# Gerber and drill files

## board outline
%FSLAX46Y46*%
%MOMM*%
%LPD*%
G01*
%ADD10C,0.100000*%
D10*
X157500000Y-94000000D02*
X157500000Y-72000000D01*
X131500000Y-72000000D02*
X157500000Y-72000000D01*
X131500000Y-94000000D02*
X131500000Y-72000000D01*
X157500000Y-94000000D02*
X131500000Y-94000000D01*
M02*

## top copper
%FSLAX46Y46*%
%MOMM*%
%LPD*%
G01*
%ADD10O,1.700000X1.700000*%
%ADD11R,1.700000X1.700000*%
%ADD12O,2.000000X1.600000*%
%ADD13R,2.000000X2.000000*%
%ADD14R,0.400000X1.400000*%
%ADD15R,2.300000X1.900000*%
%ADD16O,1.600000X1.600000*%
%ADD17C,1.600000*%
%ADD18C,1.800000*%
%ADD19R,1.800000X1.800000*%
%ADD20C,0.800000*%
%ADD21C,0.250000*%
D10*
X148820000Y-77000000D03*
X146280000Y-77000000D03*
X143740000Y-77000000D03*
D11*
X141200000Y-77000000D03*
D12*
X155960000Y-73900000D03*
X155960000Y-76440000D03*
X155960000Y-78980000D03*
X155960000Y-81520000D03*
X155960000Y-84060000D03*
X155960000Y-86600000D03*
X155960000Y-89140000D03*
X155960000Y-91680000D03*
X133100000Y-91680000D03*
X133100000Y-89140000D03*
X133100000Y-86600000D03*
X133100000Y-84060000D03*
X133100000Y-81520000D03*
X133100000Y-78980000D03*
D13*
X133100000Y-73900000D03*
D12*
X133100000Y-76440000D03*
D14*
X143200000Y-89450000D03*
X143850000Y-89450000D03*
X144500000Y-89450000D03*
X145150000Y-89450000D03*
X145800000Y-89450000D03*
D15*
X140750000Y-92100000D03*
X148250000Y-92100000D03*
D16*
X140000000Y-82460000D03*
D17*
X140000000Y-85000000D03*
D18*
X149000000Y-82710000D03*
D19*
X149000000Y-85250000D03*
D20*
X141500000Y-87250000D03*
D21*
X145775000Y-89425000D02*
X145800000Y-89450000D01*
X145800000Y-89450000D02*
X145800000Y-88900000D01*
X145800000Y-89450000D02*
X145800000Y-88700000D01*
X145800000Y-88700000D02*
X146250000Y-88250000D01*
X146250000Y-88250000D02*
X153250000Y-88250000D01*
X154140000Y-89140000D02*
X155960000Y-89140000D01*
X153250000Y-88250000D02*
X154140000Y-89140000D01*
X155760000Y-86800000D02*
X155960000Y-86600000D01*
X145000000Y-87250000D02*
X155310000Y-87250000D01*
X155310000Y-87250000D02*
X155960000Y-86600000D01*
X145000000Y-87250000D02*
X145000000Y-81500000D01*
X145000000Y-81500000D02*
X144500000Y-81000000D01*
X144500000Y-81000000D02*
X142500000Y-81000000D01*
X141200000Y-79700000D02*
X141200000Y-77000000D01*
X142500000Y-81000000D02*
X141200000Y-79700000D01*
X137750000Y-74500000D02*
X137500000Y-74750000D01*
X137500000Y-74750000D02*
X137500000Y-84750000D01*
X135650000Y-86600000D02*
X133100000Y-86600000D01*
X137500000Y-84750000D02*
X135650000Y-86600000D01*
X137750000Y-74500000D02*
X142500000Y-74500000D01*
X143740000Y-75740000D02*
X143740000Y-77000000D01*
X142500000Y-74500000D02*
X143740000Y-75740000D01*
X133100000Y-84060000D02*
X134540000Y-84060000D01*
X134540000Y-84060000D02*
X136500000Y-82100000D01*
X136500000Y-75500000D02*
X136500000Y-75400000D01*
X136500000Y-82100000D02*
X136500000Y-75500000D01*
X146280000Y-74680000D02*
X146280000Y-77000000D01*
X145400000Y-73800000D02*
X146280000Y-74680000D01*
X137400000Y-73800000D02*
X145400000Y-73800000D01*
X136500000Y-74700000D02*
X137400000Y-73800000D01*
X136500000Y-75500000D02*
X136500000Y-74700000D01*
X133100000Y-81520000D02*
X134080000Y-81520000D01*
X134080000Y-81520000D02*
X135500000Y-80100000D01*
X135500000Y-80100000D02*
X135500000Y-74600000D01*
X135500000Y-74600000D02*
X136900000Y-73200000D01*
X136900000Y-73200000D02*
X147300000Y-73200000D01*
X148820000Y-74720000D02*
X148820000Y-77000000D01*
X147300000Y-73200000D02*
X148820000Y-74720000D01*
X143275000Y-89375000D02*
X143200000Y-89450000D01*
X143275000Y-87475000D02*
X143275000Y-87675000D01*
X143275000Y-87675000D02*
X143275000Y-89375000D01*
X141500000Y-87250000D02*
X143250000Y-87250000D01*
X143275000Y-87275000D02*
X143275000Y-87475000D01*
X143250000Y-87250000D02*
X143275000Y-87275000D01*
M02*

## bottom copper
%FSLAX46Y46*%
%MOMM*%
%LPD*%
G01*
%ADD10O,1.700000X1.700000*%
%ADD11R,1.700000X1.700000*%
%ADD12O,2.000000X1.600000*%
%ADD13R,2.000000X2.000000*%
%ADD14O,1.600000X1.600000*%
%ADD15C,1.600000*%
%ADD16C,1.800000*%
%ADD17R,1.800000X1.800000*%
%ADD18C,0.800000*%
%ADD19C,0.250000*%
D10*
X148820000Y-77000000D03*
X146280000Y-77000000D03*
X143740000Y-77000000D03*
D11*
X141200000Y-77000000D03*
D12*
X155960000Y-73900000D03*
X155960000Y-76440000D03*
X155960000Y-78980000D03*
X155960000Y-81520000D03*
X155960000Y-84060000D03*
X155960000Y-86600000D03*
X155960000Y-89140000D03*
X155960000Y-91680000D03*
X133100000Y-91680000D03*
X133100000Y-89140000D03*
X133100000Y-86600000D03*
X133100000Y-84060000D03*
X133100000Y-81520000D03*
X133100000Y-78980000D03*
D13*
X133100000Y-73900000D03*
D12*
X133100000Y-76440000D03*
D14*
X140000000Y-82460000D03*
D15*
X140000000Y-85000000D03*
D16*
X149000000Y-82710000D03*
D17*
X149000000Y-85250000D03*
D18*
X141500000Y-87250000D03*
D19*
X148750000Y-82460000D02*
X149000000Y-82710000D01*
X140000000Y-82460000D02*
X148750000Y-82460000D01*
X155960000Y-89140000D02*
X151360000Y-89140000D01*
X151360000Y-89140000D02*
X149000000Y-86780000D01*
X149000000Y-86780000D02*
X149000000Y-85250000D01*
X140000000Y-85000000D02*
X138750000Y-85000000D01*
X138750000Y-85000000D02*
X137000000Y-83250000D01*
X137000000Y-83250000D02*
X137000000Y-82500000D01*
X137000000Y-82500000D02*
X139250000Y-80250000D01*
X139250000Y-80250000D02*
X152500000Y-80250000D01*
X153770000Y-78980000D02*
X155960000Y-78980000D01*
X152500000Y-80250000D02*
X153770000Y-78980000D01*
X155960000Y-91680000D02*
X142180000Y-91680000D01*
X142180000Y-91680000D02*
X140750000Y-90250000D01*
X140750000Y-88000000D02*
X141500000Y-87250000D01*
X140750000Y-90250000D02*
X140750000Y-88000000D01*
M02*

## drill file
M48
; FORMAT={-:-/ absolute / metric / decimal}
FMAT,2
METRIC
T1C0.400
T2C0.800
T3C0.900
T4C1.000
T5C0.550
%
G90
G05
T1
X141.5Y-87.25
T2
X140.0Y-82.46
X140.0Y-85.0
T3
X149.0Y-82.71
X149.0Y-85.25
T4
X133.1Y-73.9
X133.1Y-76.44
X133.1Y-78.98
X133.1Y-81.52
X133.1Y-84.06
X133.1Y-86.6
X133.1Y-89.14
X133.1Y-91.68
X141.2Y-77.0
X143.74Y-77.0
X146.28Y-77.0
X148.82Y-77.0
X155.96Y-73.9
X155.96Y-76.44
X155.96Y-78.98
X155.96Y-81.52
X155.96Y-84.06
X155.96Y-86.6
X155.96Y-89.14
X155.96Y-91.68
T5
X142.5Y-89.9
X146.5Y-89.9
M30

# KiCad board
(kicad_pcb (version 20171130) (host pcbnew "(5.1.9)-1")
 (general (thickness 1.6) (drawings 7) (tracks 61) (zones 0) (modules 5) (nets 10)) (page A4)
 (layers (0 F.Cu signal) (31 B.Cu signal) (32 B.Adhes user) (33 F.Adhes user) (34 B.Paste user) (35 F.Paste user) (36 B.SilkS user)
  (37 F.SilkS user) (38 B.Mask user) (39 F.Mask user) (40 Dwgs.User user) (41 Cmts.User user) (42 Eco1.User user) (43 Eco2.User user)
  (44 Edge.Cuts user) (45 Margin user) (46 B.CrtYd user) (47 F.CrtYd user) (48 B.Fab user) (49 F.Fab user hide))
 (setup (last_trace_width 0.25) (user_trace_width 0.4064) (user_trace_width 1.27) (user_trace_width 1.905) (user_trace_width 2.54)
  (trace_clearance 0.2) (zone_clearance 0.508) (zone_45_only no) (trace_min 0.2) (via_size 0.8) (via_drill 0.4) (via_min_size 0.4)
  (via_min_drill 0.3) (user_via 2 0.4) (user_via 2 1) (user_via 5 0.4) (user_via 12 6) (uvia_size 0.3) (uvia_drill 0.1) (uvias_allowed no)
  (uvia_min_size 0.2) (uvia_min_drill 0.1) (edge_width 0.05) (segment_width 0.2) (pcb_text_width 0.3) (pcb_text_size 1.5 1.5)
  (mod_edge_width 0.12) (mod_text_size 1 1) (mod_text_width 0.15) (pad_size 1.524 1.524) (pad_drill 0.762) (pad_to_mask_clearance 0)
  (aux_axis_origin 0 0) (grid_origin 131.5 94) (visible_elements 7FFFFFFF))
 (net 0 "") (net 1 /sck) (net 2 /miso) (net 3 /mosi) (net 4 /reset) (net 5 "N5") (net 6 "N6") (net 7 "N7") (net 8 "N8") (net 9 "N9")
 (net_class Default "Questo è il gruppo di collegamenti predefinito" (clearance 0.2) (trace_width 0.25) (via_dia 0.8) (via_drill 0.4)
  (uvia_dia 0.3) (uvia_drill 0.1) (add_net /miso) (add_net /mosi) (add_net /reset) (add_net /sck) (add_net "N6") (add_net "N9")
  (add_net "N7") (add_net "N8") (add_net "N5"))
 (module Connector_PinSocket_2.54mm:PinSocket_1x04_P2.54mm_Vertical (layer F.Cu) (at 141.2 77 90)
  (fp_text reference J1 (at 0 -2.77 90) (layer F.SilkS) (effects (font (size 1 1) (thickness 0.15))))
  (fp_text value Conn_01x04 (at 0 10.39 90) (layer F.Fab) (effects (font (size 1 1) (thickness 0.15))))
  (pad 4 thru_hole oval (at 0 7.62 90) (size 1.7 1.7) (drill 1) (layers *.Cu *.Mask) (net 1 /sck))
  (pad 3 thru_hole oval (at 0 5.08 90) (size 1.7 1.7) (drill 1) (layers *.Cu *.Mask) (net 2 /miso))
  (pad 2 thru_hole oval (at 0 2.54 90) (size 1.7 1.7) (drill 1) (layers *.Cu *.Mask) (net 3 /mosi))
  (pad 1 thru_hole rect (at 0 0 90) (size 1.7 1.7) (drill 1) (layers *.Cu *.Mask) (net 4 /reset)))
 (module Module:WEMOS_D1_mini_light (layer F.Cu) (at 133.1 73.9)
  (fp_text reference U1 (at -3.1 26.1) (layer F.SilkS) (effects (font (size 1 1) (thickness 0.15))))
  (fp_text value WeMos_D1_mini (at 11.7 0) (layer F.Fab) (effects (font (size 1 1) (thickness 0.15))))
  (pad 16 thru_hole oval (at 22.86 0) (size 2 1.6) (drill 1) (layers *.Cu *.Mask))
  (pad 15 thru_hole oval (at 22.86 2.54) (size 2 1.6) (drill 1) (layers *.Cu *.Mask))
  (pad 14 thru_hole oval (at 22.86 5.08) (size 2 1.6) (drill 1) (layers *.Cu *.Mask) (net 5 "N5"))
  (pad 13 thru_hole oval (at 22.86 7.62) (size 2 1.6) (drill 1) (layers *.Cu *.Mask))
  (pad 12 thru_hole oval (at 22.86 10.16) (size 2 1.6) (drill 1) (layers *.Cu *.Mask))
  (pad 11 thru_hole oval (at 22.86 12.7) (size 2 1.6) (drill 1) (layers *.Cu *.Mask) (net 4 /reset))
  (pad 10 thru_hole oval (at 22.86 15.24) (size 2 1.6) (drill 1) (layers *.Cu *.Mask) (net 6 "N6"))
  (pad 9 thru_hole oval (at 22.86 17.78) (size 2 1.6) (drill 1) (layers *.Cu *.Mask) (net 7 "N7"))
  (pad 8 thru_hole oval (at 0 17.78) (size 2 1.6) (drill 1) (layers *.Cu *.Mask))
  (pad 7 thru_hole oval (at 0 15.24) (size 2 1.6) (drill 1) (layers *.Cu *.Mask))
  (pad 6 thru_hole oval (at 0 12.7) (size 2 1.6) (drill 1) (layers *.Cu *.Mask) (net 3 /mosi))
  (pad 5 thru_hole oval (at 0 10.16) (size 2 1.6) (drill 1) (layers *.Cu *.Mask) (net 2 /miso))
  (pad 4 thru_hole oval (at 0 7.62) (size 2 1.6) (drill 1) (layers *.Cu *.Mask) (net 1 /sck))
  (pad 3 thru_hole oval (at 0 5.08) (size 2 1.6) (drill 1) (layers *.Cu *.Mask))
  (pad 1 thru_hole rect (at 0 0) (size 2 2) (drill 1) (layers *.Cu *.Mask))
  (pad 2 thru_hole oval (at 0 2.54) (size 2 1.6) (drill 1) (layers *.Cu *.Mask)))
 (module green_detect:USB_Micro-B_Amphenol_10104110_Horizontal (layer F.Cu) (at 144.5 91)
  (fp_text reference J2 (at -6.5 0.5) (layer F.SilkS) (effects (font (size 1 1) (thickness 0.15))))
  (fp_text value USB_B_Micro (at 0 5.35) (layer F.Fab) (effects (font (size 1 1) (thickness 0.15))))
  (pad "" np_thru_hole circle (at 2 -1.1) (size 0.55 0.55) (drill 0.55) (layers *.Cu *.Mask))
  (pad "" np_thru_hole circle (at -2 -1.1) (size 0.55 0.55) (drill 0.55) (layers *.Cu *.Mask))
  (pad 1 smd rect (at -1.3 -1.55) (size 0.4 1.4) (layers F.Cu F.Paste F.Mask) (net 7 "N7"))
  (pad 2 smd rect (at -0.65 -1.55) (size 0.4 1.4) (layers F.Cu F.Paste F.Mask))
  (pad 3 smd rect (at 0 -1.55) (size 0.4 1.4) (layers F.Cu F.Paste F.Mask))
  (pad 4 smd rect (at 0.65 -1.55) (size 0.4 1.4) (layers F.Cu F.Paste F.Mask))
  (pad 5 smd rect (at 1.3 -1.55) (size 0.4 1.4) (layers F.Cu F.Paste F.Mask) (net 6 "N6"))
  (pad 6 smd rect (at -3.75 1.1) (size 2.3 1.9) (layers F.Cu F.Paste F.Mask) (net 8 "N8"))
  (pad 6 smd rect (at 3.75 1.1) (size 2.3 1.9) (layers F.Cu F.Paste F.Mask) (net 8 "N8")))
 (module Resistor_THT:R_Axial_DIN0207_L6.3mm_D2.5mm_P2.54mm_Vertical (layer F.Cu) (at 140 85 90)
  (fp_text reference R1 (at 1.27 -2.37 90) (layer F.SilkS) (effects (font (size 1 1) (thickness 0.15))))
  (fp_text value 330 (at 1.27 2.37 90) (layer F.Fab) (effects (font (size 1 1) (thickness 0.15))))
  (pad 2 thru_hole oval (at 2.54 0 90) (size 1.6 1.6) (drill 0.8) (layers *.Cu *.Mask) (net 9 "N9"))
  (pad 1 thru_hole circle (at 0 0 90) (size 1.6 1.6) (drill 0.8) (layers *.Cu *.Mask) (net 5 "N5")))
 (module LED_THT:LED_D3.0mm (layer F.Cu) (at 149 85.25 90)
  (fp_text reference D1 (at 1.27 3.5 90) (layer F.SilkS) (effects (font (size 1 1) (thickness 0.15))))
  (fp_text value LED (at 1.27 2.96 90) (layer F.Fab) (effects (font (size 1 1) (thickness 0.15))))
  (pad 2 thru_hole circle (at 2.54 0 90) (size 1.8 1.8) (drill 0.9) (layers *.Cu *.Mask) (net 9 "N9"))
  (pad 1 thru_hole rect (at 0 0 90) (size 1.8 1.8) (drill 0.9) (layers *.Cu *.Mask) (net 6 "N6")))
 (gr_line (start 157.5 94) (end 157.5 72) (layer Edge.Cuts) (width 0.1))
 (gr_line (start 131.5 72) (end 157.5 72) (layer Edge.Cuts) (width 0.1))
 (gr_line (start 131.5 94) (end 131.5 72) (layer Edge.Cuts) (width 0.1))
 (gr_line (start 157.5 94) (end 131.5 94) (layer Edge.Cuts) (width 0.1))
 (segment (start 148.75 82.46) (end 149 82.71) (width 0.25) (layer B.Cu) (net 9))
 (segment (start 140 82.46) (end 148.75 82.46) (width 0.25) (layer B.Cu) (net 9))
 (segment (start 145.775 89.425) (end 145.8 89.45) (width 0.25) (layer F.Cu) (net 6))
 (segment (start 145.8 89.45) (end 145.8 88.9) (width 0.25) (layer F.Cu) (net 6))
 (segment (start 145.8 89.45) (end 145.8 88.7) (width 0.25) (layer F.Cu) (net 6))
 (segment (start 145.8 88.7) (end 146.25 88.25) (width 0.25) (layer F.Cu) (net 6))
 (segment (start 146.25 88.25) (end 153.25 88.25) (width 0.25) (layer F.Cu) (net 6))
 (segment (start 154.14 89.14) (end 155.96 89.14) (width 0.25) (layer F.Cu) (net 6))
 (segment (start 153.25 88.25) (end 154.14 89.14) (width 0.25) (layer F.Cu) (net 6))
 (segment (start 155.96 89.14) (end 151.36 89.14) (width 0.25) (layer B.Cu) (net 6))
 (segment (start 151.36 89.14) (end 149 86.78) (width 0.25) (layer B.Cu) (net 6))
 (segment (start 149 86.78) (end 149 85.25) (width 0.25) (layer B.Cu) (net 6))
 (segment (start 140 85) (end 138.75 85) (width 0.25) (layer B.Cu) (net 5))
 (segment (start 138.75 85) (end 137 83.25) (width 0.25) (layer B.Cu) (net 5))
 (segment (start 137 83.25) (end 137 82.5) (width 0.25) (layer B.Cu) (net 5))
 (segment (start 137 82.5) (end 139.25 80.25) (width 0.25) (layer B.Cu) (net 5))
 (segment (start 139.25 80.25) (end 152.5 80.25) (width 0.25) (layer B.Cu) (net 5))
 (segment (start 153.77 78.98) (end 155.96 78.98) (width 0.25) (layer B.Cu) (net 5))
 (segment (start 152.5 80.25) (end 153.77 78.98) (width 0.25) (layer B.Cu) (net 5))
 (segment (start 155.76 86.8) (end 155.96 86.6) (width 0.25) (layer F.Cu) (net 4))
 (segment (start 145 87.25) (end 155.31 87.25) (width 0.25) (layer F.Cu) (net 4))
 (segment (start 155.31 87.25) (end 155.96 86.6) (width 0.25) (layer F.Cu) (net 4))
 (segment (start 145 87.25) (end 145 81.5) (width 0.25) (layer F.Cu) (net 4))
 (segment (start 145 81.5) (end 144.5 81) (width 0.25) (layer F.Cu) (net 4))
 (segment (start 144.5 81) (end 142.5 81) (width 0.25) (layer F.Cu) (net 4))
 (segment (start 141.2 79.7) (end 141.2 77) (width 0.25) (layer F.Cu) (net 4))
 (segment (start 142.5 81) (end 141.2 79.7) (width 0.25) (layer F.Cu) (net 4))
 (segment (start 137.75 74.5) (end 137.5 74.75) (width 0.25) (layer F.Cu) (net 3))
 (segment (start 137.5 74.75) (end 137.5 84.75) (width 0.25) (layer F.Cu) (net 3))
 (segment (start 135.65 86.6) (end 133.1 86.6) (width 0.25) (layer F.Cu) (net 3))
 (segment (start 137.5 84.75) (end 135.65 86.6) (width 0.25) (layer F.Cu) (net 3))
 (segment (start 137.75 74.5) (end 142.5 74.5) (width 0.25) (layer F.Cu) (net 3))
 (segment (start 143.74 75.74) (end 143.74 77) (width 0.25) (layer F.Cu) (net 3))
 (segment (start 142.5 74.5) (end 143.74 75.74) (width 0.25) (layer F.Cu) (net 3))
 (segment (start 133.1 84.06) (end 134.54 84.06) (width 0.25) (layer F.Cu) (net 2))
 (segment (start 134.54 84.06) (end 136.5 82.1) (width 0.25) (layer F.Cu) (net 2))
 (segment (start 136.5 75.5) (end 136.5 75.4) (width 0.25) (layer F.Cu) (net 2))
 (segment (start 136.5 82.1) (end 136.5 75.5) (width 0.25) (layer F.Cu) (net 2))
 (segment (start 146.28 74.68) (end 146.28 77) (width 0.25) (layer F.Cu) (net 2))
 (segment (start 145.4 73.8) (end 146.28 74.68) (width 0.25) (layer F.Cu) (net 2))
 (segment (start 137.4 73.8) (end 145.4 73.8) (width 0.25) (layer F.Cu) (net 2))
 (segment (start 136.5 74.7) (end 137.4 73.8) (width 0.25) (layer F.Cu) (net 2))
 (segment (start 136.5 75.5) (end 136.5 74.7) (width 0.25) (layer F.Cu) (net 2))
 (segment (start 133.1 81.52) (end 134.08 81.52) (width 0.25) (layer F.Cu) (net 1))
 (segment (start 134.08 81.52) (end 135.5 80.1) (width 0.25) (layer F.Cu) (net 1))
 (segment (start 135.5 80.1) (end 135.5 74.6) (width 0.25) (layer F.Cu) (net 1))
 (segment (start 135.5 74.6) (end 136.9 73.2) (width 0.25) (layer F.Cu) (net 1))
 (segment (start 136.9 73.2) (end 147.3 73.2) (width 0.25) (layer F.Cu) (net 1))
 (segment (start 148.82 74.72) (end 148.82 77) (width 0.25) (layer F.Cu) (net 1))
 (segment (start 147.3 73.2) (end 148.82 74.72) (width 0.25) (layer F.Cu) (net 1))
 (segment (start 143.275 89.375) (end 143.2 89.45) (width 0.25) (layer F.Cu) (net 7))
 (segment (start 143.275 87.475) (end 143.275 87.675) (width 0.25) (layer F.Cu) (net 7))
 (segment (start 143.275 87.675) (end 143.275 89.375) (width 0.25) (layer F.Cu) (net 7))
 (segment (start 155.96 91.68) (end 142.18 91.68) (width 0.25) (layer B.Cu) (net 7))
 (segment (start 142.18 91.68) (end 140.75 90.25) (width 0.25) (layer B.Cu) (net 7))
 (via (at 141.5 87.25) (size 0.8) (drill 0.4) (layers F.Cu B.Cu) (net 7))
 (segment (start 140.75 88) (end 141.5 87.25) (width 0.25) (layer B.Cu) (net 7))
 (segment (start 140.75 90.25) (end 140.75 88) (width 0.25) (layer B.Cu) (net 7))
 (segment (start 141.5 87.25) (end 143.25 87.25) (width 0.25) (layer F.Cu) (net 7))
 (segment (start 143.275 87.275) (end 143.275 87.475) (width 0.25) (layer F.Cu) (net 7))
 (segment (start 143.25 87.25) (end 143.275 87.275) (width 0.25) (layer F.Cu) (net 7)))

